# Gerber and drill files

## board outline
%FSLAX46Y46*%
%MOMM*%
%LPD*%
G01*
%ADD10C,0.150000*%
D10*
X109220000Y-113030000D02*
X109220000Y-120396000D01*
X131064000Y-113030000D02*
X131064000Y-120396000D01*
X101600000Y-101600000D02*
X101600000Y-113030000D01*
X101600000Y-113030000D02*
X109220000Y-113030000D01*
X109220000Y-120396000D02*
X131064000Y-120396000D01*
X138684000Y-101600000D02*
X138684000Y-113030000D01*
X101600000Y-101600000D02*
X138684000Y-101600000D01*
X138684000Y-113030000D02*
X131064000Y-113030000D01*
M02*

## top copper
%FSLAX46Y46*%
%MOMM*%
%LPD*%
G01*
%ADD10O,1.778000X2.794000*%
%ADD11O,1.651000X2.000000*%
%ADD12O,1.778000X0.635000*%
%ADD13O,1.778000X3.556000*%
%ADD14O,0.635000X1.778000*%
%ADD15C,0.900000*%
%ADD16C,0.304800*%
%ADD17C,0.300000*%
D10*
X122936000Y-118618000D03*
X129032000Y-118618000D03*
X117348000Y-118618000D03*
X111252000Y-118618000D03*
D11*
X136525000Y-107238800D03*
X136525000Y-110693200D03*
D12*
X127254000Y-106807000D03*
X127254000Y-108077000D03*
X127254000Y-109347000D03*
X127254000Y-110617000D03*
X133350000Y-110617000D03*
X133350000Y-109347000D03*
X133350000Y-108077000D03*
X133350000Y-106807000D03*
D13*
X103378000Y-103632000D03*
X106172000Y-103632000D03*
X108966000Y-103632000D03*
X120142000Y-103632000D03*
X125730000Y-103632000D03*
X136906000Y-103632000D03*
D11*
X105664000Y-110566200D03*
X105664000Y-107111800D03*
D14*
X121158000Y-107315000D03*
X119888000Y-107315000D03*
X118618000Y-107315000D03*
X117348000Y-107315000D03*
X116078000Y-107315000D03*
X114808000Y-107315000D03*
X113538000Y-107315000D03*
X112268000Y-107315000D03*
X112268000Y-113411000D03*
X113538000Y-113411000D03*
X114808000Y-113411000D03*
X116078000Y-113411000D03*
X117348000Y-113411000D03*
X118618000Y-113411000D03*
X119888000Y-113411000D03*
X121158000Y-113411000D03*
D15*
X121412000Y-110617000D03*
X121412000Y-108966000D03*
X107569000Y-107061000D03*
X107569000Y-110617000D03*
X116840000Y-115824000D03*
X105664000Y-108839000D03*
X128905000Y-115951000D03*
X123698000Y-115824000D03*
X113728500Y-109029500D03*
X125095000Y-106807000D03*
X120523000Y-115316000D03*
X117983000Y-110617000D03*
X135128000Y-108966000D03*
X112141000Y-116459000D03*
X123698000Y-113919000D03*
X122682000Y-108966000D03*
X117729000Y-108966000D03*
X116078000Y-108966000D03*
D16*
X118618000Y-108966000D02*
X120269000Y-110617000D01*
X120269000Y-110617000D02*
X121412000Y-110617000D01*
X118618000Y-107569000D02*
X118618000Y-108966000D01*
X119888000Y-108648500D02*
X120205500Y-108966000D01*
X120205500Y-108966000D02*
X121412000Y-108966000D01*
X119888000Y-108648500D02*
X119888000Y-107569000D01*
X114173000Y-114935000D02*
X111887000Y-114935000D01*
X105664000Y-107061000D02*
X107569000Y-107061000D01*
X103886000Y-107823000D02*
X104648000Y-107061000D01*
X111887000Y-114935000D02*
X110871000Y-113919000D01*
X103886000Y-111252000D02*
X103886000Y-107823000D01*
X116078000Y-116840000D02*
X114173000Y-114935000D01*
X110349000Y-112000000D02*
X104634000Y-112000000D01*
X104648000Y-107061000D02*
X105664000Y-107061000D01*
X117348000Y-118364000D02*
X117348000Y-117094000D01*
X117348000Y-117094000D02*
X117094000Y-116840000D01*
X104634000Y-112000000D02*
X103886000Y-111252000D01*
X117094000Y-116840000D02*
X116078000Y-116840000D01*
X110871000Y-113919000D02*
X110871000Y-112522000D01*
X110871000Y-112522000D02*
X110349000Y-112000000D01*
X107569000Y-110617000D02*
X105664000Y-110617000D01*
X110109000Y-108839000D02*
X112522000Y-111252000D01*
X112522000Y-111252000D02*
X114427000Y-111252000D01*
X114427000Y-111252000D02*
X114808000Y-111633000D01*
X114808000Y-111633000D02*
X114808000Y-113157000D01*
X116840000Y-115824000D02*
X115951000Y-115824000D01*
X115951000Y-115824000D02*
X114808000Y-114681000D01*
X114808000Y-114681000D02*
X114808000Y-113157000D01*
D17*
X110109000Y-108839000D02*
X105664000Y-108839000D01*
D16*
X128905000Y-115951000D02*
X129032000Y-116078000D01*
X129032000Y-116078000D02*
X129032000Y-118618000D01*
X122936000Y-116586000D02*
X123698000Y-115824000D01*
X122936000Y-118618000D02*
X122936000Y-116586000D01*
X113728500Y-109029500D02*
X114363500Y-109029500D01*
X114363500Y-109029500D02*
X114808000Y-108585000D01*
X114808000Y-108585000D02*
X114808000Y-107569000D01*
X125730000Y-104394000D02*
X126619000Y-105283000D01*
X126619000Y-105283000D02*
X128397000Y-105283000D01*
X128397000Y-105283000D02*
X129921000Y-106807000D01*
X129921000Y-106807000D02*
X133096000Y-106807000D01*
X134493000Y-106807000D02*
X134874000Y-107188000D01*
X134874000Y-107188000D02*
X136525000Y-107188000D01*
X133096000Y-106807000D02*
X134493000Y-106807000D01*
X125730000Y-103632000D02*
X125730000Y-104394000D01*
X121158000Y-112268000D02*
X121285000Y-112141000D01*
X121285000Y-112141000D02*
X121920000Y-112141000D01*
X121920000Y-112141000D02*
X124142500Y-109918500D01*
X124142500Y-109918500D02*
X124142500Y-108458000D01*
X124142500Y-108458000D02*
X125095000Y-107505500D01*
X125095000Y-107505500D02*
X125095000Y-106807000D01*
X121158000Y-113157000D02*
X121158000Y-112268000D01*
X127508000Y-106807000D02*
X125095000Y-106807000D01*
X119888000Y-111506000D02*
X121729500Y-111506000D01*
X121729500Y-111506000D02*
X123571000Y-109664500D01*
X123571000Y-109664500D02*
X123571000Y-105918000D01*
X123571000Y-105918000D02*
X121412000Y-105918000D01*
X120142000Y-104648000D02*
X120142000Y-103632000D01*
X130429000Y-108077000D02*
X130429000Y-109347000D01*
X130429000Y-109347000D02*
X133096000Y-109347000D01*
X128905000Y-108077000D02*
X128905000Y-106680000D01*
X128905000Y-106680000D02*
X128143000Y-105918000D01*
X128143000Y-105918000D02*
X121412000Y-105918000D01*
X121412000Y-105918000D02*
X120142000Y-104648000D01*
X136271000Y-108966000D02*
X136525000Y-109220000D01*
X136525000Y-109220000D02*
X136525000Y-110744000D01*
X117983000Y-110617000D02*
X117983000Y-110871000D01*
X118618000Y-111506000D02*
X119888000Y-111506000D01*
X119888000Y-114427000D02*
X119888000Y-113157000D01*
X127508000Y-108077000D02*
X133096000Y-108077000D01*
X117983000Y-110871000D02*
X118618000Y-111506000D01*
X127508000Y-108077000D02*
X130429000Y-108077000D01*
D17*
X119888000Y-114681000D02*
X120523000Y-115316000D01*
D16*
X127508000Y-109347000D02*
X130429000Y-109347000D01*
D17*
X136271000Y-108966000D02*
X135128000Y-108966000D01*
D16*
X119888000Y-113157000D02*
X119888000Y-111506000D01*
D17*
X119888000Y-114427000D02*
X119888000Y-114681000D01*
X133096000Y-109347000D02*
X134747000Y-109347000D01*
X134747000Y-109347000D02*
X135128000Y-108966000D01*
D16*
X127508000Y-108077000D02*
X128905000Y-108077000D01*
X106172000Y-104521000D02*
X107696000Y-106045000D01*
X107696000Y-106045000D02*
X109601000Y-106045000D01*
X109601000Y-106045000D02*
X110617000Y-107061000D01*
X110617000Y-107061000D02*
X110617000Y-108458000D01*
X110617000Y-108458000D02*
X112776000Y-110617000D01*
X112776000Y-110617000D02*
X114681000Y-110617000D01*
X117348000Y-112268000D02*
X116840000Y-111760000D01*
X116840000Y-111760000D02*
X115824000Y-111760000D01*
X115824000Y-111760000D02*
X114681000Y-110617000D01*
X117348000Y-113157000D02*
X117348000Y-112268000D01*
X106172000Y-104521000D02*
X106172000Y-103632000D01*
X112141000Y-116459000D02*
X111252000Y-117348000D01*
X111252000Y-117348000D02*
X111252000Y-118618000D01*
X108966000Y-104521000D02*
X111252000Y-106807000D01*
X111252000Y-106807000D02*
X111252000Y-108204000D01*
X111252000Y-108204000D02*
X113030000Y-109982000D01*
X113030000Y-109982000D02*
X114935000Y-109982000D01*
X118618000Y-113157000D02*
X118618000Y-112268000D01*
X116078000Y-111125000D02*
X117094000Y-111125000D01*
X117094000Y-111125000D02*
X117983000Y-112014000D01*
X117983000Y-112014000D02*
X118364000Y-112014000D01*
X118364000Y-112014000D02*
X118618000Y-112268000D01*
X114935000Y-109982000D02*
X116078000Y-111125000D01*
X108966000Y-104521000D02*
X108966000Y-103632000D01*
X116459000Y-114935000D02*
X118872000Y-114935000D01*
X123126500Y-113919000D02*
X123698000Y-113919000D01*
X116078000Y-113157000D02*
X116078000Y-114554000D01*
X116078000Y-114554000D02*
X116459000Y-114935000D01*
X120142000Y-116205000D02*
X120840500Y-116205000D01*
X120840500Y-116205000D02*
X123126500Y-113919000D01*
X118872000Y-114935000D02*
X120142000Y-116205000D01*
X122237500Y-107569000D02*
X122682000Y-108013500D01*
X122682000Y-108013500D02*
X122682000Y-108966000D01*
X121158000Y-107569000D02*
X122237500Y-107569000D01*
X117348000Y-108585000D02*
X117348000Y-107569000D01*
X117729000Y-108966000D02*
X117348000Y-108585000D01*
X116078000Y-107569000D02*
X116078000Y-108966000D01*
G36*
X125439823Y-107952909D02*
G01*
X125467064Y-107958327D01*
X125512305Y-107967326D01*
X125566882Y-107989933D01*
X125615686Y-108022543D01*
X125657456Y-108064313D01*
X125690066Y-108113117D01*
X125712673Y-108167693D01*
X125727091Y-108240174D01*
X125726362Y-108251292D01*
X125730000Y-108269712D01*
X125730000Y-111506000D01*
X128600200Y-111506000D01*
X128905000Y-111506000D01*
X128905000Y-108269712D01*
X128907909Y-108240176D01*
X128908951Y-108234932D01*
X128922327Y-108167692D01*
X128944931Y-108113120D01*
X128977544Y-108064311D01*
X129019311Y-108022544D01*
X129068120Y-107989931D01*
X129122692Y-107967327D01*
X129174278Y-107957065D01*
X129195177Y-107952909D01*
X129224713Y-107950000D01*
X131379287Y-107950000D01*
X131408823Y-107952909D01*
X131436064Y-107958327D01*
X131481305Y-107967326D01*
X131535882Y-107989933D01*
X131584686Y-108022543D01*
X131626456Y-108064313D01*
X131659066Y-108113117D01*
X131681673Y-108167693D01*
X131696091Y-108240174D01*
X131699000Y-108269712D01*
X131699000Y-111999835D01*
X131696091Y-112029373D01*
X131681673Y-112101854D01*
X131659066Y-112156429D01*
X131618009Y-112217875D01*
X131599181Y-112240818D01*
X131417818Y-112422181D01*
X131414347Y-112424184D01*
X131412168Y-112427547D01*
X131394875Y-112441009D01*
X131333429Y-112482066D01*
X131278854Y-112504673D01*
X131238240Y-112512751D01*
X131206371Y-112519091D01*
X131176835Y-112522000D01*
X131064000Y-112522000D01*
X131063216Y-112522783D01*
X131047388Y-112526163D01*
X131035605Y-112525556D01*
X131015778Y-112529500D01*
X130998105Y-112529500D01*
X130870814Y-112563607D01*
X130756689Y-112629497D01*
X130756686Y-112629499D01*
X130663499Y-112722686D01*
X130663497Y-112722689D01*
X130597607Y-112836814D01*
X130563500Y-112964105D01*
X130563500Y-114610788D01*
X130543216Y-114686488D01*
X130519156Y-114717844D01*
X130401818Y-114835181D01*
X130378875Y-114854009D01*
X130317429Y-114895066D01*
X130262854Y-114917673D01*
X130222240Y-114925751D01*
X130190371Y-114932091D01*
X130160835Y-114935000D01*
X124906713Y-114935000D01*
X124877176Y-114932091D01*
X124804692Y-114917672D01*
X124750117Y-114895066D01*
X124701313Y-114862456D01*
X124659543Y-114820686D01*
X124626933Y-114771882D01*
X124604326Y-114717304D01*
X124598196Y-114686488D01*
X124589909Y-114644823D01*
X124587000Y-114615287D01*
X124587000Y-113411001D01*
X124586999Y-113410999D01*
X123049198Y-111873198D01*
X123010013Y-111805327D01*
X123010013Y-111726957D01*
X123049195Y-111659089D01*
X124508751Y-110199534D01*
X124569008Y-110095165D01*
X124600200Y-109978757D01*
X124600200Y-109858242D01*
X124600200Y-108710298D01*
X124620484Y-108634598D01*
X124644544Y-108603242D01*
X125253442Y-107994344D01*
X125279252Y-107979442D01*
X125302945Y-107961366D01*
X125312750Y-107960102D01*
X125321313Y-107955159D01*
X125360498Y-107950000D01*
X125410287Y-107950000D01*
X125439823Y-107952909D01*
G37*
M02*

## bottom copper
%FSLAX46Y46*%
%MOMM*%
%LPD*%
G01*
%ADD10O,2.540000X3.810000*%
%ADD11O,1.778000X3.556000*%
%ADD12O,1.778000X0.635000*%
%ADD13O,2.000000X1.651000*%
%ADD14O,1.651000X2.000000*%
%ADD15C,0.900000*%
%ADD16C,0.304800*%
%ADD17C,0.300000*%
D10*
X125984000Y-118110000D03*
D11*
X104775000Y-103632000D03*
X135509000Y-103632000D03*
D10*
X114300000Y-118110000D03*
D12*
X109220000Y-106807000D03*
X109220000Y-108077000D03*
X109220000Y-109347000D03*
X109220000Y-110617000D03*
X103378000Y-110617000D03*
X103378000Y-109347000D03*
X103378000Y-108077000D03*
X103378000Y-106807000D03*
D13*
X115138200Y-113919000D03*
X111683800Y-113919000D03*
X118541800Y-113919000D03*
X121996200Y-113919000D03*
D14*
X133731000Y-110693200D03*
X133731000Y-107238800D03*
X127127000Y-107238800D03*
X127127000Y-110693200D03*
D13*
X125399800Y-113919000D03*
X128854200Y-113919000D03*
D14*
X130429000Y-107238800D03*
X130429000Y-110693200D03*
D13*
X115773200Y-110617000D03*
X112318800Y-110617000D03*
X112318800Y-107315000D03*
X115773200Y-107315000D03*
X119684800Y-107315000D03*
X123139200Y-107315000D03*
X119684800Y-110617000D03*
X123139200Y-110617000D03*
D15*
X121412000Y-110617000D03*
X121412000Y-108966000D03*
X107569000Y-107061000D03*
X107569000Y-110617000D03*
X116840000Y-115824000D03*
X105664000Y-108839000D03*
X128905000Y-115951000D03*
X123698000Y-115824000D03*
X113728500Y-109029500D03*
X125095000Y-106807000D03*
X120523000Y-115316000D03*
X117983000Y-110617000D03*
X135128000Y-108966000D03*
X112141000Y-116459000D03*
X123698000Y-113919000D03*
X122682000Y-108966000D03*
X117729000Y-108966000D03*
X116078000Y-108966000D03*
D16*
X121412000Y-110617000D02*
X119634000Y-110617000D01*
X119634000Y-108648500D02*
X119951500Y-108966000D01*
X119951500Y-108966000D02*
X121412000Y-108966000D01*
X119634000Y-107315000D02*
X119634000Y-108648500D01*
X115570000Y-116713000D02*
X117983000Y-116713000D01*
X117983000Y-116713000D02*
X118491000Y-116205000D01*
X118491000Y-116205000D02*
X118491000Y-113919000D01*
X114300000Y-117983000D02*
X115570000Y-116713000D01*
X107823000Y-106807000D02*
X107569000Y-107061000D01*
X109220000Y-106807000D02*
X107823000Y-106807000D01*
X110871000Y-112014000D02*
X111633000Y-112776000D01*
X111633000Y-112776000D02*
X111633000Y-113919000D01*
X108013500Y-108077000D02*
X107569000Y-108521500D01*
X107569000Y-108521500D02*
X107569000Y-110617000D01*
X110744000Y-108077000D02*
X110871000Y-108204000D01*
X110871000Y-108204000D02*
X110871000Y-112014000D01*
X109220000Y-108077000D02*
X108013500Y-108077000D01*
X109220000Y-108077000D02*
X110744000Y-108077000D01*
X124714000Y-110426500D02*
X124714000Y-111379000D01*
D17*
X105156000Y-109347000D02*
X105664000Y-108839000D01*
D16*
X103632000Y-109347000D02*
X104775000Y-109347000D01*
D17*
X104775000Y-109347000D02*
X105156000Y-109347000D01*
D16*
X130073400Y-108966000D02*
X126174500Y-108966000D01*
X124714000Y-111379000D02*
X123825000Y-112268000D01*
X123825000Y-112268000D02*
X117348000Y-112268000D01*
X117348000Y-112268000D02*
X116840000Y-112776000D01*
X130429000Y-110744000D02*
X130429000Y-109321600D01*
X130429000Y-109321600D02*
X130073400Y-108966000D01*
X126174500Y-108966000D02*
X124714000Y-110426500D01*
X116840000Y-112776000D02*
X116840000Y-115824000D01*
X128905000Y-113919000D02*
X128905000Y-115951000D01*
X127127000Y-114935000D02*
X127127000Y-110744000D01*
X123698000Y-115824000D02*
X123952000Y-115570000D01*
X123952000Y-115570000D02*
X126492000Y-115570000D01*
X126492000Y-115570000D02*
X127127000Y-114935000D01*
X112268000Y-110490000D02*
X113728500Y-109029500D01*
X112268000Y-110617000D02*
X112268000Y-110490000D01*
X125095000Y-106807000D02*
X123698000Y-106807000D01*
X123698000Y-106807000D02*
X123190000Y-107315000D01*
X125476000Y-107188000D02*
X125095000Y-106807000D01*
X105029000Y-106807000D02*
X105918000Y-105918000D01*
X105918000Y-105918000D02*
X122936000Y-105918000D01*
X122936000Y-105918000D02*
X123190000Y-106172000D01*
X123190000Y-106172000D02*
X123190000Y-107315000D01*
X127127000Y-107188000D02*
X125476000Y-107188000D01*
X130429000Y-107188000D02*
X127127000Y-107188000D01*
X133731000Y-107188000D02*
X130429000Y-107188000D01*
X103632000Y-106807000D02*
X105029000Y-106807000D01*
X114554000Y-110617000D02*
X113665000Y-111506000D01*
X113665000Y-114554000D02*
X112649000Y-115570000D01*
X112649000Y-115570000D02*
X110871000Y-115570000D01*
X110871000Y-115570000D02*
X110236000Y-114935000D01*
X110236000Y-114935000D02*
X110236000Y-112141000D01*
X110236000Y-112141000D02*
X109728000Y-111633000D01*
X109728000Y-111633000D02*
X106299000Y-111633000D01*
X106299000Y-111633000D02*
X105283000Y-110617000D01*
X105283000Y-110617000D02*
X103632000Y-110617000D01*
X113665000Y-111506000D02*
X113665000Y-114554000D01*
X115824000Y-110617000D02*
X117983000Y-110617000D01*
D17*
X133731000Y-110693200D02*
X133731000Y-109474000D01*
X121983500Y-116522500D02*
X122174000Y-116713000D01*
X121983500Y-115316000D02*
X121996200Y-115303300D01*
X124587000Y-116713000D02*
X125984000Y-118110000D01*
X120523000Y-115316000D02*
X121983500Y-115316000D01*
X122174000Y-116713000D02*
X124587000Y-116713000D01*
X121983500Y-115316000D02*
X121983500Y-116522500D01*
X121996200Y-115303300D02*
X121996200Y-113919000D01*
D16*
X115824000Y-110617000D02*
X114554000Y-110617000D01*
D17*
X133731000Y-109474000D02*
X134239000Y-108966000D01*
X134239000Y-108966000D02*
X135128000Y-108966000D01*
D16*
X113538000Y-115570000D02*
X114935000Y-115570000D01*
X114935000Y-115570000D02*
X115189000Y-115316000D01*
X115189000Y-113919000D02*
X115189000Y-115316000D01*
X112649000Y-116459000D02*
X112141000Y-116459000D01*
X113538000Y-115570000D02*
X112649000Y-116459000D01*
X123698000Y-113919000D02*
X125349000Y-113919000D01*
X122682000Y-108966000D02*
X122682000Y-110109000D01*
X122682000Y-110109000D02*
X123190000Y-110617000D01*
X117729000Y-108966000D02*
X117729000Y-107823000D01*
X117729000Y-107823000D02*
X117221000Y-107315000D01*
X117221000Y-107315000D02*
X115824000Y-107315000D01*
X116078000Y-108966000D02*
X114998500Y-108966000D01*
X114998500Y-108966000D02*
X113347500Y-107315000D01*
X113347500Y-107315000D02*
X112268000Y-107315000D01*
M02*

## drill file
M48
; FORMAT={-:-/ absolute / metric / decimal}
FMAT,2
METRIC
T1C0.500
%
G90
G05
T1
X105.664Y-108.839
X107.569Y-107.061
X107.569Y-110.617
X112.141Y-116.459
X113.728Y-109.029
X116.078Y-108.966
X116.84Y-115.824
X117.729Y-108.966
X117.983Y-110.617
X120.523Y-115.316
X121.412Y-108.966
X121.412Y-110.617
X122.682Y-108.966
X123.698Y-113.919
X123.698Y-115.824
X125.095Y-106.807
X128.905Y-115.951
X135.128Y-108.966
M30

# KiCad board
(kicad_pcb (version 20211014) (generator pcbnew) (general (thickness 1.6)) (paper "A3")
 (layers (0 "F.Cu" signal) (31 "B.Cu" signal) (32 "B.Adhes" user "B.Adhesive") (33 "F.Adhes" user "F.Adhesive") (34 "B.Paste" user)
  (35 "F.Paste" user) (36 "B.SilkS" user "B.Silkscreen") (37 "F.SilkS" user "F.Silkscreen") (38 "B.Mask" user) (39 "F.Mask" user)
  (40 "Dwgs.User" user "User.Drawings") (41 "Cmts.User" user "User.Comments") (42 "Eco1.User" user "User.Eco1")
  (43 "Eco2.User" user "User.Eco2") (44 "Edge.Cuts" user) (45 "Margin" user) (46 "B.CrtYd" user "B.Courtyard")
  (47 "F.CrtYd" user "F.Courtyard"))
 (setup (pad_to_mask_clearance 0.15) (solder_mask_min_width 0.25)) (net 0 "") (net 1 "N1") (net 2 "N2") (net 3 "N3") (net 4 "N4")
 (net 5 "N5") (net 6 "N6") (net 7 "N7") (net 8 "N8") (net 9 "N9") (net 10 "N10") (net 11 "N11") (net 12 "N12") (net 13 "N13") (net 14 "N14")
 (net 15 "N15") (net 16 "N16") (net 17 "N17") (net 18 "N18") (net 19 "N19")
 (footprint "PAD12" (layer "F.Cu") (at 125.984 118.11)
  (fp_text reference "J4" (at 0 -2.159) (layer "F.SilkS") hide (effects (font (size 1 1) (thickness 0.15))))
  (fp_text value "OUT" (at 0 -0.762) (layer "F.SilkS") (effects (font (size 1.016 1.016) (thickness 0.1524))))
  (pad "1" smd oval locked (at 0 0) (size 2.54 3.81) (layers "B.Cu" "B.Mask") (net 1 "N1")))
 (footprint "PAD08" (layer "F.Cu") (at 122.936 118.618)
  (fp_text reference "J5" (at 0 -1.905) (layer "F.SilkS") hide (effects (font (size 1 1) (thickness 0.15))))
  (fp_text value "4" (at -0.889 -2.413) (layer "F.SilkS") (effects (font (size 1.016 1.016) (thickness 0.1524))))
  (pad "1" smd oval locked (at 0 0) (size 1.778 2.794) (layers "F.Cu" "F.Paste" "F.Mask") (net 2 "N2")))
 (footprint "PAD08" (layer "F.Cu") (at 129.032 118.618)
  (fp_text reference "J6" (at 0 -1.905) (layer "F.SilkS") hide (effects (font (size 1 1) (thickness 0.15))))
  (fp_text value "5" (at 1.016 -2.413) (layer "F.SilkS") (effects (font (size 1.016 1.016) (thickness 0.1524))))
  (pad "1" smd oval locked (at 0 0) (size 1.778 2.794) (layers "F.Cu" "F.Paste" "F.Mask") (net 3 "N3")))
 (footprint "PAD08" (layer "F.Cu") (at 117.348 118.618)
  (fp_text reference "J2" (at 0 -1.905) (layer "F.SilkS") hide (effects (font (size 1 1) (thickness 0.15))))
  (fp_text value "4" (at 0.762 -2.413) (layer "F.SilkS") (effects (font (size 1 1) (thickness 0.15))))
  (pad "1" smd oval locked (at 0 0) (size 1.778 2.794) (layers "F.Cu" "F.Paste" "F.Mask") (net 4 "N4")))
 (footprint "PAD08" (layer "F.Cu") (at 111.252 118.618)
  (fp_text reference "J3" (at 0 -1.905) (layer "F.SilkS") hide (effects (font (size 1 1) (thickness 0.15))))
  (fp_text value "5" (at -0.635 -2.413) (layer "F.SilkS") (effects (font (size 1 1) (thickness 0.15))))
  (pad "1" smd oval locked (at 0 0) (size 1.778 2.794) (layers "F.Cu" "F.Paste" "F.Mask") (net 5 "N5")))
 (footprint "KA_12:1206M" (layer "F.Cu") (at 136.525 108.966 -90)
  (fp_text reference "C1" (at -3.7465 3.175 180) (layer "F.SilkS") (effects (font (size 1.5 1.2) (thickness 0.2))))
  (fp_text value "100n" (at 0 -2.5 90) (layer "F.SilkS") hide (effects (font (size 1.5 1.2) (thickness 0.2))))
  (pad "1" smd oval locked (at -1.7272 0 270) (size 2 1.651) (layers "F.Cu" "F.Paste" "F.Mask") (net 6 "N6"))
  (pad "2" smd oval locked (at 1.7272 0 270) (size 2 1.651) (layers "F.Cu" "F.Paste" "F.Mask") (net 1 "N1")))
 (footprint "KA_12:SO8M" (layer "F.Cu") (at 130.302 108.712 -90)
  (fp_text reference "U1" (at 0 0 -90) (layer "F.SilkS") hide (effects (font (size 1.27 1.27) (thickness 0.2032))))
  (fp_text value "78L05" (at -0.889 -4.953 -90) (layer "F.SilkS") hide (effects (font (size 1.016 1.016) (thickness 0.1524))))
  (pad "1" smd oval (at -1.905 2.794 270) (size 0.635 1.778) (drill (offset 0 0.254)) (layers "F.Cu" "F.Paste" "F.Mask") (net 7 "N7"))
  (pad "2" smd oval (at -0.635 2.794 270) (size 0.635 1.778) (drill (offset 0 0.254)) (layers "F.Cu" "F.Paste" "F.Mask") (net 1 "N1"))
  (pad "3" smd oval (at 0.635 2.794 270) (size 0.635 1.778) (drill (offset 0 0.254)) (layers "F.Cu" "F.Paste" "F.Mask") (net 1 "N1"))
  (pad "4" smd oval (at 1.905 2.794 270) (size 0.635 1.778) (drill (offset 0 0.254)) (layers "F.Cu" "F.Paste" "F.Mask"))
  (pad "5" smd oval (at 1.905 -2.794 270) (size 0.635 1.778) (drill (offset 0 -0.254)) (layers "F.Cu" "F.Paste" "F.Mask"))
  (pad "6" smd oval (at 0.635 -2.794 270) (size 0.635 1.778) (drill (offset 0 -0.254)) (layers "F.Cu" "F.Paste" "F.Mask") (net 1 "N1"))
  (pad "7" smd oval (at -0.635 -2.794 270) (size 0.635 1.778) (drill (offset 0 -0.254)) (layers "F.Cu" "F.Paste" "F.Mask") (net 1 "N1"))
  (pad "8" smd oval (at -1.905 -2.794 270) (size 0.635 1.778) (drill (offset 0 -0.254)) (layers "F.Cu" "F.Paste" "F.Mask") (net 6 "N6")))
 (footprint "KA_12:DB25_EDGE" (layer "F.Cu") (at 120.142 103.632)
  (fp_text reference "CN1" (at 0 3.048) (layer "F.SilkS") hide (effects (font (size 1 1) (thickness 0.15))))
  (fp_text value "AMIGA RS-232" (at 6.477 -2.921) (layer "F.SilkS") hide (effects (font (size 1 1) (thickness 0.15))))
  (pad "1" smd oval locked (at -16.764 0) (size 1.778 3.556) (layers "F.Cu" "F.Paste" "F.Mask"))
  (pad "2" smd oval locked (at -13.97 0) (size 1.778 3.556) (layers "F.Cu" "F.Paste" "F.Mask") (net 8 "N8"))
  (pad "3" smd oval locked (at -11.176 0) (size 1.778 3.556) (layers "F.Cu" "F.Paste" "F.Mask") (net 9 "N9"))
  (pad "7" smd oval locked (at 0 0) (size 1.778 3.556) (layers "F.Cu" "F.Paste" "F.Mask") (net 1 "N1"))
  (pad "9" smd oval locked (at 5.588 0) (size 1.778 3.556) (layers "F.Cu" "F.Paste" "F.Mask") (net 6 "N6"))
  (pad "13" smd oval locked (at 16.764 0) (size 1.778 3.556) (layers "F.Cu" "F.Paste" "F.Mask"))
  (pad "14" smd oval locked (at -15.367 0) (size 1.778 3.556) (layers "B.Cu" "B.Paste" "B.Mask"))
  (pad "25" smd oval locked (at 15.367 0) (size 1.778 3.556) (layers "B.Cu" "B.Paste" "B.Mask")))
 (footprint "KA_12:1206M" (layer "F.Cu") (at 105.664 108.839 90)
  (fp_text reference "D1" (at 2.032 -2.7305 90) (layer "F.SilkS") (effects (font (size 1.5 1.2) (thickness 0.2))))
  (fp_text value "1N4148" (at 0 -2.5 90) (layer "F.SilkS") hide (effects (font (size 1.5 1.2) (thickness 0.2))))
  (pad "1" smd oval locked (at -1.7272 0 90) (size 2 1.651) (layers "F.Cu" "F.Paste" "F.Mask") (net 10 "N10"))
  (pad "2" smd oval locked (at 1.7272 0 90) (size 2 1.651) (layers "F.Cu" "F.Paste" "F.Mask") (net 4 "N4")))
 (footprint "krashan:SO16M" (layer "F.Cu") (at 116.713 110.363 180)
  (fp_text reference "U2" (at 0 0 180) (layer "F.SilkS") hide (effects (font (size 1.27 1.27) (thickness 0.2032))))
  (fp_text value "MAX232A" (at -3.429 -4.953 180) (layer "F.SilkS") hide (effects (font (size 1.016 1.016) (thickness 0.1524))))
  (pad "1" smd oval (at -4.445 2.794 180) (size 0.635 1.778) (drill (offset 0 0.254)) (layers "F.Cu" "F.Paste" "F.Mask") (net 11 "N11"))
  (pad "2" smd oval (at -3.175 2.794 180) (size 0.635 1.778) (drill (offset 0 0.254)) (layers "F.Cu" "F.Paste" "F.Mask") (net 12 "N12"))
  (pad "3" smd oval (at -1.905 2.794 180) (size 0.635 1.778) (drill (offset 0 0.254)) (layers "F.Cu" "F.Paste" "F.Mask") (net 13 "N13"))
  (pad "4" smd oval (at -0.635 2.794 180) (size 0.635 1.778) (drill (offset 0 0.254)) (layers "F.Cu" "F.Paste" "F.Mask") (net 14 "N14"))
  (pad "5" smd oval (at 0.635 2.794 180) (size 0.635 1.778) (drill (offset 0 0.254)) (layers "F.Cu" "F.Paste" "F.Mask") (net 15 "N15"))
  (pad "6" smd oval (at 1.905 2.794 180) (size 0.635 1.778) (drill (offset 0 0.254)) (layers "F.Cu" "F.Paste" "F.Mask") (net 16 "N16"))
  (pad "7" smd oval (at 3.175 2.794 180) (size 0.635 1.778) (drill (offset 0 0.254)) (layers "F.Cu" "F.Paste" "F.Mask"))
  (pad "8" smd oval (at 4.445 2.794 180) (size 0.635 1.778) (drill (offset 0 0.254)) (layers "F.Cu" "F.Paste" "F.Mask"))
  (pad "9" smd oval (at 4.445 -2.794 180) (size 0.635 1.778) (drill (offset 0 -0.254)) (layers "F.Cu" "F.Paste" "F.Mask"))
  (pad "10" smd oval (at 3.175 -2.794 180) (size 0.635 1.778) (drill (offset 0 -0.254)) (layers "F.Cu" "F.Paste" "F.Mask"))
  (pad "11" smd oval (at 1.905 -2.794 180) (size 0.635 1.778) (drill (offset 0 -0.254)) (layers "F.Cu" "F.Paste" "F.Mask") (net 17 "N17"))
  (pad "12" smd oval (at 0.635 -2.794 180) (size 0.635 1.778) (drill (offset 0 -0.254)) (layers "F.Cu" "F.Paste" "F.Mask") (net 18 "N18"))
  (pad "13" smd oval (at -0.635 -2.794 180) (size 0.635 1.778) (drill (offset 0 -0.254)) (layers "F.Cu" "F.Paste" "F.Mask") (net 8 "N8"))
  (pad "14" smd oval (at -1.905 -2.794 180) (size 0.635 1.778) (drill (offset 0 -0.254)) (layers "F.Cu" "F.Paste" "F.Mask") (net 9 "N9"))
  (pad "15" smd oval (at -3.175 -2.794 180) (size 0.635 1.778) (drill (offset 0 -0.254)) (layers "F.Cu" "F.Paste" "F.Mask") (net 1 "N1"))
  (pad "16" smd oval (at -4.445 -2.794 180) (size 0.635 1.778) (drill (offset 0 -0.254)) (layers "F.Cu" "F.Paste" "F.Mask") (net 7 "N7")))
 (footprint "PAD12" (layer "F.Cu") (at 114.3 118.11)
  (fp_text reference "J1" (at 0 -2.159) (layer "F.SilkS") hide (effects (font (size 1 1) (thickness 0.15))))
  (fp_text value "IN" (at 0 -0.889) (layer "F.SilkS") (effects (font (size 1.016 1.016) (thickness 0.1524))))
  (pad "1" smd oval locked (at 0 0) (size 2.54 3.81) (layers "B.Cu" "B.Mask") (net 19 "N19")))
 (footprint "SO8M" (layer "B.Cu") (at 106.426 108.712 -90)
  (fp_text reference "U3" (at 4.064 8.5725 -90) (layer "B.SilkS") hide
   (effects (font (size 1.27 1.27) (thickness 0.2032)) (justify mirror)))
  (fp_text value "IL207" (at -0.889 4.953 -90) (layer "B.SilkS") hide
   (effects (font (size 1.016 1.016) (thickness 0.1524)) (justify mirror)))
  (pad "1" smd oval locked (at -1.905 -2.794 270) (size 0.635 1.778) (layers "B.Cu" "B.Paste" "B.Mask") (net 4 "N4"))
  (pad "2" smd oval locked (at -0.635 -2.794 270) (size 0.635 1.778) (layers "B.Cu" "B.Paste" "B.Mask") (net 10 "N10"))
  (pad "3" smd oval locked (at 0.635 -2.794 270) (size 0.635 1.778) (layers "B.Cu" "B.Paste" "B.Mask"))
  (pad "4" smd oval locked (at 1.905 -2.794 270) (size 0.635 1.778) (layers "B.Cu" "B.Paste" "B.Mask"))
  (pad "5" smd oval locked (at 1.905 2.794 270) (size 0.635 1.778) (drill (offset 0 0.254)) (layers "B.Cu" "B.Paste" "B.Mask") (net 1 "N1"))
  (pad "6" smd oval locked (at 0.635 2.794 270) (size 0.635 1.778) (drill (offset 0 0.254)) (layers "B.Cu" "B.Paste" "B.Mask")
   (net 17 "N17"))
  (pad "7" smd oval locked (at -0.635 2.794 270) (size 0.635 1.778) (drill (offset 0 0.254)) (layers "B.Cu" "B.Paste" "B.Mask"))
  (pad "8" smd oval locked (at -1.905 2.794 270) (size 0.635 1.778) (drill (offset 0 0.254)) (layers "B.Cu" "B.Paste" "B.Mask") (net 7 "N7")))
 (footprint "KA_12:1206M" (layer "B.Cu") (at 113.411 113.919 180)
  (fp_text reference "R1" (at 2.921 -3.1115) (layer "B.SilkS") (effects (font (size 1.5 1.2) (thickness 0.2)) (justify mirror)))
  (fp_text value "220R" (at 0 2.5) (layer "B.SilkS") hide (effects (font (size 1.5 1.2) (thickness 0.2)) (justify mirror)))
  (pad "1" smd oval locked (at -1.7272 0 180) (size 2 1.651) (layers "B.Cu" "B.Paste" "B.Mask") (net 5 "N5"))
  (pad "2" smd oval locked (at 1.7272 0 180) (size 2 1.651) (layers "B.Cu" "B.Paste" "B.Mask") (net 10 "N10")))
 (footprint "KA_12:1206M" (layer "B.Cu") (at 120.269 113.919)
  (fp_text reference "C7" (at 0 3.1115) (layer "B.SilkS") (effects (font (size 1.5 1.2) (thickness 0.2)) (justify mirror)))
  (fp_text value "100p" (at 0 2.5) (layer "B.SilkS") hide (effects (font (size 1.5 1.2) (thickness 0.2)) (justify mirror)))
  (pad "1" smd oval locked (at -1.7272 0) (size 2 1.651) (layers "B.Cu" "B.Paste" "B.Mask") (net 19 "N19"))
  (pad "2" smd oval locked (at 1.7272 0) (size 2 1.651) (layers "B.Cu" "B.Paste" "B.Mask") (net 1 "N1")))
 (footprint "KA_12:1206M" (layer "B.Cu") (at 133.731 108.966 90)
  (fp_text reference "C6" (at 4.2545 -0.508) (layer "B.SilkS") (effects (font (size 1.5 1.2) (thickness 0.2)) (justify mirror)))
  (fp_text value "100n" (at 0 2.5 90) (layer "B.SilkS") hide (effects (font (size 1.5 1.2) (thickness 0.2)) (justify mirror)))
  (pad "1" smd oval locked (at -1.7272 0 90) (size 2 1.651) (layers "B.Cu" "B.Paste" "B.Mask") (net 1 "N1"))
  (pad "2" smd oval locked (at 1.7272 0 90) (size 2 1.651) (layers "B.Cu" "B.Paste" "B.Mask") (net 7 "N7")))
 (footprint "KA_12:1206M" (layer "B.Cu") (at 127.127 108.966 -90)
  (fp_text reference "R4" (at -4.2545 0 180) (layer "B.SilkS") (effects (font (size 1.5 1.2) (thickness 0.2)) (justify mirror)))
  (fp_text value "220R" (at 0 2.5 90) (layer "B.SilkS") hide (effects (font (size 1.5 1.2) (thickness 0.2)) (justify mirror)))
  (pad "1" smd oval locked (at -1.7272 0 270) (size 2 1.651) (layers "B.Cu" "B.Paste" "B.Mask") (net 7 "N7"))
  (pad "2" smd oval locked (at 1.7272 0 270) (size 2 1.651) (layers "B.Cu" "B.Paste" "B.Mask") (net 2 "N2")))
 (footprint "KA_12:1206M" (layer "B.Cu") (at 127.127 113.919)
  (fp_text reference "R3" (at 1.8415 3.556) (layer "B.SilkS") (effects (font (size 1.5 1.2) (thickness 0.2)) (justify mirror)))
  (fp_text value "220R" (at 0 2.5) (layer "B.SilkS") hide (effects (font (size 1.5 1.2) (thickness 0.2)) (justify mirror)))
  (pad "1" smd oval locked (at -1.7272 0) (size 2 1.651) (layers "B.Cu" "B.Paste" "B.Mask") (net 18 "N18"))
  (pad "2" smd oval locked (at 1.7272 0) (size 2 1.651) (layers "B.Cu" "B.Paste" "B.Mask") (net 3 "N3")))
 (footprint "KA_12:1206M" (layer "B.Cu") (at 130.429 108.966 -90)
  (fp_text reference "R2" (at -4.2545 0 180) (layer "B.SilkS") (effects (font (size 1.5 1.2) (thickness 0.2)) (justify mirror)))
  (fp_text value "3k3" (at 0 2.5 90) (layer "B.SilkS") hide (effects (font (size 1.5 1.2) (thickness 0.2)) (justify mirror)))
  (pad "1" smd oval locked (at -1.7272 0 270) (size 2 1.651) (layers "B.Cu" "B.Paste" "B.Mask") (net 7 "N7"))
  (pad "2" smd oval locked (at 1.7272 0 270) (size 2 1.651) (layers "B.Cu" "B.Paste" "B.Mask") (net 17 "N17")))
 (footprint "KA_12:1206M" (layer "B.Cu") (at 114.046 110.617 180)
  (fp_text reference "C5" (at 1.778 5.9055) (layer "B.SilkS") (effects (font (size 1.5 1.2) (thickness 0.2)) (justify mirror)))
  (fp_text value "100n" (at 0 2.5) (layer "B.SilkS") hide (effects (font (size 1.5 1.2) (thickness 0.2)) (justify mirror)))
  (pad "1" smd oval locked (at -1.7272 0 180) (size 2 1.651) (layers "B.Cu" "B.Paste" "B.Mask") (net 1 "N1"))
  (pad "2" smd oval locked (at 1.7272 0 180) (size 2 1.651) (layers "B.Cu" "B.Paste" "B.Mask") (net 16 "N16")))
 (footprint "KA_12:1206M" (layer "B.Cu") (at 114.046 107.315)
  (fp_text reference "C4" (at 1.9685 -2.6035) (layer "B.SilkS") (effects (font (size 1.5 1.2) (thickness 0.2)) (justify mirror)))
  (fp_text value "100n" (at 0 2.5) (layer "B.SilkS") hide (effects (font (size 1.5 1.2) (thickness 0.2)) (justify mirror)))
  (pad "1" smd oval locked (at -1.7272 0) (size 2 1.651) (layers "B.Cu" "B.Paste" "B.Mask") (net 15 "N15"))
  (pad "2" smd oval locked (at 1.7272 0) (size 2 1.651) (layers "B.Cu" "B.Paste" "B.Mask") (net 14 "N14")))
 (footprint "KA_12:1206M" (layer "B.Cu") (at 121.412 107.315)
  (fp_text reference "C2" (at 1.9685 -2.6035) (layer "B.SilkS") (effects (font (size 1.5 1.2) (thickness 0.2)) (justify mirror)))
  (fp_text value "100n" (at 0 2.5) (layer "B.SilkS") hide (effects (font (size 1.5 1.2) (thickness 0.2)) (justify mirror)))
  (pad "1" smd oval locked (at -1.7272 0) (size 2 1.651) (layers "B.Cu" "B.Paste" "B.Mask") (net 12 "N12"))
  (pad "2" smd oval locked (at 1.7272 0) (size 2 1.651) (layers "B.Cu" "B.Paste" "B.Mask") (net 7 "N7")))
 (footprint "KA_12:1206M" (layer "B.Cu") (at 121.412 110.617)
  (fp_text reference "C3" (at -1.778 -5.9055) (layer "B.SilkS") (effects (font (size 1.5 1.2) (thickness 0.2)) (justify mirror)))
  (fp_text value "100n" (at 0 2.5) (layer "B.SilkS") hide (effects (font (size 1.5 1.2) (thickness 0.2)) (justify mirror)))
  (pad "1" smd oval locked (at -1.7272 0) (size 2 1.651) (layers "B.Cu" "B.Paste" "B.Mask") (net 13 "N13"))
  (pad "2" smd oval locked (at 1.7272 0) (size 2 1.651) (layers "B.Cu" "B.Paste" "B.Mask") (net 11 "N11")))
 (gr_line (start 109.22 113.03) (end 109.22 120.396) (layer "Edge.Cuts") (width 0.15))
 (gr_line (start 131.064 113.03) (end 131.064 120.396) (layer "Edge.Cuts") (width 0.15))
 (gr_line (start 101.6 101.6) (end 101.6 113.03) (layer "Edge.Cuts") (width 0.15))
 (gr_line (start 101.6 113.03) (end 109.22 113.03) (layer "Edge.Cuts") (width 0.15))
 (gr_line (start 109.22 120.396) (end 131.064 120.396) (layer "Edge.Cuts") (width 0.15))
 (gr_line (start 138.684 101.6) (end 138.684 113.03) (layer "Edge.Cuts") (width 0.15))
 (gr_line (start 101.6 101.6) (end 138.684 101.6) (layer "Edge.Cuts") (width 0.15))
 (gr_line (start 138.684 113.03) (end 131.064 113.03) (layer "Edge.Cuts") (width 0.15))
 (segment (start 118.618 108.966) (end 120.269 110.617) (width 0.3048) (layer "F.Cu") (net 13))
 (segment (start 120.269 110.617) (end 121.412 110.617) (width 0.3048) (layer "F.Cu") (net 13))
 (segment (start 118.618 107.569) (end 118.618 108.966) (width 0.3048) (layer "F.Cu") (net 13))
 (via (at 121.412 110.617) (size 0.9) (drill 0.5) (layers "F.Cu" "B.Cu") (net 13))
 (segment (start 121.412 110.617) (end 119.634 110.617) (width 0.3048) (layer "B.Cu") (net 13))
 (segment (start 119.888 108.6485) (end 120.2055 108.966) (width 0.3048) (layer "F.Cu") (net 12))
 (segment (start 120.2055 108.966) (end 121.412 108.966) (width 0.3048) (layer "F.Cu") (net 12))
 (segment (start 119.888 108.6485) (end 119.888 107.569) (width 0.3048) (layer "F.Cu") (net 12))
 (via (at 121.412 108.966) (size 0.9) (drill 0.5) (layers "F.Cu" "B.Cu") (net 12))
 (segment (start 119.634 108.6485) (end 119.9515 108.966) (width 0.3048) (layer "B.Cu") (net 12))
 (segment (start 119.9515 108.966) (end 121.412 108.966) (width 0.3048) (layer "B.Cu") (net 12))
 (segment (start 119.634 107.315) (end 119.634 108.6485) (width 0.3048) (layer "B.Cu") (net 12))
 (segment (start 115.57 116.713) (end 117.983 116.713) (width 0.3048) (layer "B.Cu") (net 19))
 (segment (start 117.983 116.713) (end 118.491 116.205) (width 0.3048) (layer "B.Cu") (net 19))
 (segment (start 118.491 116.205) (end 118.491 113.919) (width 0.3048) (layer "B.Cu") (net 19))
 (segment (start 114.3 117.983) (end 115.57 116.713) (width 0.3048) (layer "B.Cu") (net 19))
 (segment (start 114.173 114.935) (end 111.887 114.935) (width 0.3048) (layer "F.Cu") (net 4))
 (segment (start 105.664 107.061) (end 107.569 107.061) (width 0.3048) (layer "F.Cu") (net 4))
 (segment (start 103.886 107.823) (end 104.648 107.061) (width 0.3048) (layer "F.Cu") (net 4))
 (segment (start 111.887 114.935) (end 110.871 113.919) (width 0.3048) (layer "F.Cu") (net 4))
 (segment (start 103.886 111.252) (end 103.886 107.823) (width 0.3048) (layer "F.Cu") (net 4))
 (segment (start 116.078 116.84) (end 114.173 114.935) (width 0.3048) (layer "F.Cu") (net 4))
 (segment (start 110.349 112) (end 104.634 112) (width 0.3048) (layer "F.Cu") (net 4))
 (segment (start 104.648 107.061) (end 105.664 107.061) (width 0.3048) (layer "F.Cu") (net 4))
 (segment (start 117.348 118.364) (end 117.348 117.094) (width 0.3048) (layer "F.Cu") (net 4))
 (segment (start 117.348 117.094) (end 117.094 116.84) (width 0.3048) (layer "F.Cu") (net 4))
 (segment (start 104.634 112) (end 103.886 111.252) (width 0.3048) (layer "F.Cu") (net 4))
 (segment (start 117.094 116.84) (end 116.078 116.84) (width 0.3048) (layer "F.Cu") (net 4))
 (segment (start 110.871 113.919) (end 110.871 112.522) (width 0.3048) (layer "F.Cu") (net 4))
 (segment (start 110.871 112.522) (end 110.349 112) (width 0.3048) (layer "F.Cu") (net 4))
 (via (at 107.569 107.061) (size 0.9) (drill 0.5) (layers "F.Cu" "B.Cu") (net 4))
 (segment (start 107.823 106.807) (end 107.569 107.061) (width 0.3048) (layer "B.Cu") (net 4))
 (segment (start 109.22 106.807) (end 107.823 106.807) (width 0.3048) (layer "B.Cu") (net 4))
 (segment (start 107.569 110.617) (end 105.664 110.617) (width 0.3048) (layer "F.Cu") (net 10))
 (via (at 107.569 110.617) (size 0.9) (drill 0.5) (layers "F.Cu" "B.Cu") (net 10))
 (segment (start 110.871 112.014) (end 111.633 112.776) (width 0.3048) (layer "B.Cu") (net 10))
 (segment (start 111.633 112.776) (end 111.633 113.919) (width 0.3048) (layer "B.Cu") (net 10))
 (segment (start 108.0135 108.077) (end 107.569 108.5215) (width 0.3048) (layer "B.Cu") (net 10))
 (segment (start 107.569 108.5215) (end 107.569 110.617) (width 0.3048) (layer "B.Cu") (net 10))
 (segment (start 110.744 108.077) (end 110.871 108.204) (width 0.3048) (layer "B.Cu") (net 10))
 (segment (start 110.871 108.204) (end 110.871 112.014) (width 0.3048) (layer "B.Cu") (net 10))
 (segment (start 109.22 108.077) (end 108.0135 108.077) (width 0.3048) (layer "B.Cu") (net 10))
 (segment (start 109.22 108.077) (end 110.744 108.077) (width 0.3048) (layer "B.Cu") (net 10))
 (segment (start 110.109 108.839) (end 112.522 111.252) (width 0.3048) (layer "F.Cu") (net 17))
 (segment (start 112.522 111.252) (end 114.427 111.252) (width 0.3048) (layer "F.Cu") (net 17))
 (segment (start 114.427 111.252) (end 114.808 111.633) (width 0.3048) (layer "F.Cu") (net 17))
 (segment (start 114.808 111.633) (end 114.808 113.157) (width 0.3048) (layer "F.Cu") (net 17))
 (segment (start 116.84 115.824) (end 115.951 115.824) (width 0.3048) (layer "F.Cu") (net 17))
 (segment (start 115.951 115.824) (end 114.808 114.681) (width 0.3048) (layer "F.Cu") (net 17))
 (segment (start 114.808 114.681) (end 114.808 113.157) (width 0.3048) (layer "F.Cu") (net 17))
 (segment (start 110.109 108.839) (end 105.664 108.839) (width 0.3) (layer "F.Cu") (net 17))
 (via (at 116.84 115.824) (size 0.9) (drill 0.5) (layers "F.Cu" "B.Cu") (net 17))
 (via (at 105.664 108.839) (size 0.9) (drill 0.5) (layers "F.Cu" "B.Cu") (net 17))
 (segment (start 124.714 110.4265) (end 124.714 111.379) (width 0.3048) (layer "B.Cu") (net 17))
 (segment (start 105.156 109.347) (end 105.664 108.839) (width 0.3) (layer "B.Cu") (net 17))
 (segment (start 103.632 109.347) (end 104.775 109.347) (width 0.3048) (layer "B.Cu") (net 17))
 (segment (start 104.775 109.347) (end 105.156 109.347) (width 0.3) (layer "B.Cu") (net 17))
 (segment (start 130.0734 108.966) (end 126.1745 108.966) (width 0.3048) (layer "B.Cu") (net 17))
 (segment (start 124.714 111.379) (end 123.825 112.268) (width 0.3048) (layer "B.Cu") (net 17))
 (segment (start 123.825 112.268) (end 117.348 112.268) (width 0.3048) (layer "B.Cu") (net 17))
 (segment (start 117.348 112.268) (end 116.84 112.776) (width 0.3048) (layer "B.Cu") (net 17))
 (segment (start 130.429 110.744) (end 130.429 109.3216) (width 0.3048) (layer "B.Cu") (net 17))
 (segment (start 130.429 109.3216) (end 130.0734 108.966) (width 0.3048) (layer "B.Cu") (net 17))
 (segment (start 126.1745 108.966) (end 124.714 110.4265) (width 0.3048) (layer "B.Cu") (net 17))
 (segment (start 116.84 112.776) (end 116.84 115.824) (width 0.3048) (layer "B.Cu") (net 17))
 (segment (start 128.905 115.951) (end 129.032 116.078) (width 0.3048) (layer "F.Cu") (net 3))
 (segment (start 129.032 116.078) (end 129.032 118.618) (width 0.3048) (layer "F.Cu") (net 3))
 (via (at 128.905 115.951) (size 0.9) (drill 0.5) (layers "F.Cu" "B.Cu") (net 3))
 (segment (start 128.905 113.919) (end 128.905 115.951) (width 0.3048) (layer "B.Cu") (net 3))
 (segment (start 122.936 116.586) (end 123.698 115.824) (width 0.3048) (layer "F.Cu") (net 2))
 (segment (start 122.936 118.618) (end 122.936 116.586) (width 0.3048) (layer "F.Cu") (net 2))
 (via (at 123.698 115.824) (size 0.9) (drill 0.5) (layers "F.Cu" "B.Cu") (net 2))
 (segment (start 127.127 114.935) (end 127.127 110.744) (width 0.3048) (layer "B.Cu") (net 2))
 (segment (start 123.698 115.824) (end 123.952 115.57) (width 0.3048) (layer "B.Cu") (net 2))
 (segment (start 123.952 115.57) (end 126.492 115.57) (width 0.3048) (layer "B.Cu") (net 2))
 (segment (start 126.492 115.57) (end 127.127 114.935) (width 0.3048) (layer "B.Cu") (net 2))
 (segment (start 113.7285 109.0295) (end 114.3635 109.0295) (width 0.3048) (layer "F.Cu") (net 16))
 (segment (start 114.3635 109.0295) (end 114.808 108.585) (width 0.3048) (layer "F.Cu") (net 16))
 (segment (start 114.808 108.585) (end 114.808 107.569) (width 0.3048) (layer "F.Cu") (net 16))
 (via (at 113.7285 109.0295) (size 0.9) (drill 0.5) (layers "F.Cu" "B.Cu") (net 16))
 (segment (start 112.268 110.49) (end 113.7285 109.0295) (width 0.3048) (layer "B.Cu") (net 16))
 (segment (start 112.268 110.617) (end 112.268 110.49) (width 0.3048) (layer "B.Cu") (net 16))
 (segment (start 125.73 104.394) (end 126.619 105.283) (width 0.3048) (layer "F.Cu") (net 6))
 (segment (start 126.619 105.283) (end 128.397 105.283) (width 0.3048) (layer "F.Cu") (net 6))
 (segment (start 128.397 105.283) (end 129.921 106.807) (width 0.3048) (layer "F.Cu") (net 6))
 (segment (start 129.921 106.807) (end 133.096 106.807) (width 0.3048) (layer "F.Cu") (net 6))
 (segment (start 134.493 106.807) (end 134.874 107.188) (width 0.3048) (layer "F.Cu") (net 6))
 (segment (start 134.874 107.188) (end 136.525 107.188) (width 0.3048) (layer "F.Cu") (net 6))
 (segment (start 133.096 106.807) (end 134.493 106.807) (width 0.3048) (layer "F.Cu") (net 6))
 (segment (start 125.73 103.632) (end 125.73 104.394) (width 0.3048) (layer "F.Cu") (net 6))
 (segment (start 121.158 112.268) (end 121.285 112.141) (width 0.3048) (layer "F.Cu") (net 7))
 (segment (start 121.285 112.141) (end 121.92 112.141) (width 0.3048) (layer "F.Cu") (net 7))
 (segment (start 121.92 112.141) (end 124.1425 109.9185) (width 0.3048) (layer "F.Cu") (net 7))
 (segment (start 124.1425 109.9185) (end 124.1425 108.458) (width 0.3048) (layer "F.Cu") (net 7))
 (segment (start 124.1425 108.458) (end 125.095 107.5055) (width 0.3048) (layer "F.Cu") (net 7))
 (segment (start 125.095 107.5055) (end 125.095 106.807) (width 0.3048) (layer "F.Cu") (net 7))
 (segment (start 121.158 113.157) (end 121.158 112.268) (width 0.3048) (layer "F.Cu") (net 7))
 (segment (start 127.508 106.807) (end 125.095 106.807) (width 0.3048) (layer "F.Cu") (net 7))
 (via (at 125.095 106.807) (size 0.9) (drill 0.5) (layers "F.Cu" "B.Cu") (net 7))
 (segment (start 125.095 106.807) (end 123.698 106.807) (width 0.3048) (layer "B.Cu") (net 7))
 (segment (start 123.698 106.807) (end 123.19 107.315) (width 0.3048) (layer "B.Cu") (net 7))
 (segment (start 125.476 107.188) (end 125.095 106.807) (width 0.3048) (layer "B.Cu") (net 7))
 (segment (start 105.029 106.807) (end 105.918 105.918) (width 0.3048) (layer "B.Cu") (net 7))
 (segment (start 105.918 105.918) (end 122.936 105.918) (width 0.3048) (layer "B.Cu") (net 7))
 (segment (start 122.936 105.918) (end 123.19 106.172) (width 0.3048) (layer "B.Cu") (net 7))
 (segment (start 123.19 106.172) (end 123.19 107.315) (width 0.3048) (layer "B.Cu") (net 7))
 (segment (start 127.127 107.188) (end 125.476 107.188) (width 0.3048) (layer "B.Cu") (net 7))
 (segment (start 130.429 107.188) (end 127.127 107.188) (width 0.3048) (layer "B.Cu") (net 7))
 (segment (start 133.731 107.188) (end 130.429 107.188) (width 0.3048) (layer "B.Cu") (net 7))
 (segment (start 103.632 106.807) (end 105.029 106.807) (width 0.3048) (layer "B.Cu") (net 7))
 (segment (start 119.888 111.506) (end 121.7295 111.506) (width 0.3048) (layer "F.Cu") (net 1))
 (segment (start 121.7295 111.506) (end 123.571 109.6645) (width 0.3048) (layer "F.Cu") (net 1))
 (segment (start 123.571 109.6645) (end 123.571 105.918) (width 0.3048) (layer "F.Cu") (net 1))
 (segment (start 123.571 105.918) (end 121.412 105.918) (width 0.3048) (layer "F.Cu") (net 1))
 (segment (start 120.142 104.648) (end 120.142 103.632) (width 0.3048) (layer "F.Cu") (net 1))
 (segment (start 130.429 108.077) (end 130.429 109.347) (width 0.3048) (layer "F.Cu") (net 1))
 (segment (start 130.429 109.347) (end 133.096 109.347) (width 0.3048) (layer "F.Cu") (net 1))
 (segment (start 128.905 108.077) (end 128.905 106.68) (width 0.3048) (layer "F.Cu") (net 1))
 (segment (start 128.905 106.68) (end 128.143 105.918) (width 0.3048) (layer "F.Cu") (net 1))
 (segment (start 128.143 105.918) (end 121.412 105.918) (width 0.3048) (layer "F.Cu") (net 1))
 (segment (start 121.412 105.918) (end 120.142 104.648) (width 0.3048) (layer "F.Cu") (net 1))
 (segment (start 136.271 108.966) (end 136.525 109.22) (width 0.3048) (layer "F.Cu") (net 1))
 (segment (start 136.525 109.22) (end 136.525 110.744) (width 0.3048) (layer "F.Cu") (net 1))
 (segment (start 117.983 110.617) (end 117.983 110.871) (width 0.3048) (layer "F.Cu") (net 1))
 (segment (start 118.618 111.506) (end 119.888 111.506) (width 0.3048) (layer "F.Cu") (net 1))
 (segment (start 119.888 114.427) (end 119.888 113.157) (width 0.3048) (layer "F.Cu") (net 1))
 (segment (start 127.508 108.077) (end 133.096 108.077) (width 0.3048) (layer "F.Cu") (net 1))
 (segment (start 117.983 110.871) (end 118.618 111.506) (width 0.3048) (layer "F.Cu") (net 1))
 (segment (start 127.508 108.077) (end 130.429 108.077) (width 0.3048) (layer "F.Cu") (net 1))
 (segment (start 119.888 114.681) (end 120.523 115.316) (width 0.3) (layer "F.Cu") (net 1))
 (segment (start 127.508 109.347) (end 130.429 109.347) (width 0.3048) (layer "F.Cu") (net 1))
 (segment (start 136.271 108.966) (end 135.128 108.966) (width 0.3) (layer "F.Cu") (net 1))
 (segment (start 119.888 113.157) (end 119.888 111.506) (width 0.3048) (layer "F.Cu") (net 1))
 (segment (start 119.888 114.427) (end 119.888 114.681) (width 0.3) (layer "F.Cu") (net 1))
 (segment (start 133.096 109.347) (end 134.747 109.347) (width 0.3) (layer "F.Cu") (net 1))
 (segment (start 134.747 109.347) (end 135.128 108.966) (width 0.3) (layer "F.Cu") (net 1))
 (segment (start 127.508 108.077) (end 128.905 108.077) (width 0.3048) (layer "F.Cu") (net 1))
 (via (at 120.523 115.316) (size 0.9) (drill 0.5) (layers "F.Cu" "B.Cu") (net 1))
 (via (at 117.983 110.617) (size 0.9) (drill 0.5) (layers "F.Cu" "B.Cu") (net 1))
 (via (at 135.128 108.966) (size 0.9) (drill 0.5) (layers "F.Cu" "B.Cu") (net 1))
 (segment (start 114.554 110.617) (end 113.665 111.506) (width 0.3048) (layer "B.Cu") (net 1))
 (segment (start 113.665 114.554) (end 112.649 115.57) (width 0.3048) (layer "B.Cu") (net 1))
 (segment (start 112.649 115.57) (end 110.871 115.57) (width 0.3048) (layer "B.Cu") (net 1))
 (segment (start 110.871 115.57) (end 110.236 114.935) (width 0.3048) (layer "B.Cu") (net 1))
 (segment (start 110.236 114.935) (end 110.236 112.141) (width 0.3048) (layer "B.Cu") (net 1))
 (segment (start 110.236 112.141) (end 109.728 111.633) (width 0.3048) (layer "B.Cu") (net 1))
 (segment (start 109.728 111.633) (end 106.299 111.633) (width 0.3048) (layer "B.Cu") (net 1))
 (segment (start 106.299 111.633) (end 105.283 110.617) (width 0.3048) (layer "B.Cu") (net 1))
 (segment (start 105.283 110.617) (end 103.632 110.617) (width 0.3048) (layer "B.Cu") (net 1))
 (segment (start 113.665 111.506) (end 113.665 114.554) (width 0.3048) (layer "B.Cu") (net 1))
 (segment (start 115.824 110.617) (end 117.983 110.617) (width 0.3048) (layer "B.Cu") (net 1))
 (segment (start 133.731 110.6932) (end 133.731 109.474) (width 0.3) (layer "B.Cu") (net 1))
 (segment (start 121.9835 116.5225) (end 122.174 116.713) (width 0.3) (layer "B.Cu") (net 1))
 (segment (start 121.9835 115.316) (end 121.9962 115.3033) (width 0.3) (layer "B.Cu") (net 1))
 (segment (start 124.587 116.713) (end 125.984 118.11) (width 0.3) (layer "B.Cu") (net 1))
 (segment (start 120.523 115.316) (end 121.9835 115.316) (width 0.3) (layer "B.Cu") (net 1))
 (segment (start 122.174 116.713) (end 124.587 116.713) (width 0.3) (layer "B.Cu") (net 1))
 (segment (start 121.9835 115.316) (end 121.9835 116.5225) (width 0.3) (layer "B.Cu") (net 1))
 (segment (start 121.9962 115.3033) (end 121.9962 113.919) (width 0.3) (layer "B.Cu") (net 1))
 (segment (start 115.824 110.617) (end 114.554 110.617) (width 0.3048) (layer "B.Cu") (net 1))
 (segment (start 133.731 109.474) (end 134.239 108.966) (width 0.3) (layer "B.Cu") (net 1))
 (segment (start 134.239 108.966) (end 135.128 108.966) (width 0.3) (layer "B.Cu") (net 1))
 (segment (start 106.172 104.521) (end 107.696 106.045) (width 0.3048) (layer "F.Cu") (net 8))
 (segment (start 107.696 106.045) (end 109.601 106.045) (width 0.3048) (layer "F.Cu") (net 8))
 (segment (start 109.601 106.045) (end 110.617 107.061) (width 0.3048) (layer "F.Cu") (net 8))
 (segment (start 110.617 107.061) (end 110.617 108.458) (width 0.3048) (layer "F.Cu") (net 8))
 (segment (start 110.617 108.458) (end 112.776 110.617) (width 0.3048) (layer "F.Cu") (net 8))
 (segment (start 112.776 110.617) (end 114.681 110.617) (width 0.3048) (layer "F.Cu") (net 8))
 (segment (start 117.348 112.268) (end 116.84 111.76) (width 0.3048) (layer "F.Cu") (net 8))
 (segment (start 116.84 111.76) (end 115.824 111.76) (width 0.3048) (layer "F.Cu") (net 8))
 (segment (start 115.824 111.76) (end 114.681 110.617) (width 0.3048) (layer "F.Cu") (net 8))
 (segment (start 117.348 113.157) (end 117.348 112.268) (width 0.3048) (layer "F.Cu") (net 8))
 (segment (start 106.172 104.521) (end 106.172 103.632) (width 0.3048) (layer "F.Cu") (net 8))
 (segment (start 112.141 116.459) (end 111.252 117.348) (width 0.3048) (layer "F.Cu") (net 5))
 (segment (start 111.252 117.348) (end 111.252 118.618) (width 0.3048) (layer "F.Cu") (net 5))
 (via (at 112.141 116.459) (size 0.9) (drill 0.5) (layers "F.Cu" "B.Cu") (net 5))
 (segment (start 113.538 115.57) (end 114.935 115.57) (width 0.3048) (layer "B.Cu") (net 5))
 (segment (start 114.935 115.57) (end 115.189 115.316) (width 0.3048) (layer "B.Cu") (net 5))
 (segment (start 115.189 113.919) (end 115.189 115.316) (width 0.3048) (layer "B.Cu") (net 5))
 (segment (start 112.649 116.459) (end 112.141 116.459) (width 0.3048) (layer "B.Cu") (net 5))
 (segment (start 113.538 115.57) (end 112.649 116.459) (width 0.3048) (layer "B.Cu") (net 5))
 (segment (start 108.966 104.521) (end 111.252 106.807) (width 0.3048) (layer "F.Cu") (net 9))
 (segment (start 111.252 106.807) (end 111.252 108.204) (width 0.3048) (layer "F.Cu") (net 9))
 (segment (start 111.252 108.204) (end 113.03 109.982) (width 0.3048) (layer "F.Cu") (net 9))
 (segment (start 113.03 109.982) (end 114.935 109.982) (width 0.3048) (layer "F.Cu") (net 9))
 (segment (start 118.618 113.157) (end 118.618 112.268) (width 0.3048) (layer "F.Cu") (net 9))
 (segment (start 116.078 111.125) (end 117.094 111.125) (width 0.3048) (layer "F.Cu") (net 9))
 (segment (start 117.094 111.125) (end 117.983 112.014) (width 0.3048) (layer "F.Cu") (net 9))
 (segment (start 117.983 112.014) (end 118.364 112.014) (width 0.3048) (layer "F.Cu") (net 9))
 (segment (start 118.364 112.014) (end 118.618 112.268) (width 0.3048) (layer "F.Cu") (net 9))
 (segment (start 114.935 109.982) (end 116.078 111.125) (width 0.3048) (layer "F.Cu") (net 9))
 (segment (start 108.966 104.521) (end 108.966 103.632) (width 0.3048) (layer "F.Cu") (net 9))
 (segment (start 116.459 114.935) (end 118.872 114.935) (width 0.3048) (layer "F.Cu") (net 18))
 (segment (start 123.1265 113.919) (end 123.698 113.919) (width 0.3048) (layer "F.Cu") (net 18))
 (segment (start 116.078 113.157) (end 116.078 114.554) (width 0.3048) (layer "F.Cu") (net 18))
 (segment (start 116.078 114.554) (end 116.459 114.935) (width 0.3048) (layer "F.Cu") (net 18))
 (segment (start 120.142 116.205) (end 120.8405 116.205) (width 0.3048) (layer "F.Cu") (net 18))
 (segment (start 120.8405 116.205) (end 123.1265 113.919) (width 0.3048) (layer "F.Cu") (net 18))
 (segment (start 118.872 114.935) (end 120.142 116.205) (width 0.3048) (layer "F.Cu") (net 18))
 (via (at 123.698 113.919) (size 0.9) (drill 0.5) (layers "F.Cu" "B.Cu") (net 18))
 (segment (start 123.698 113.919) (end 125.349 113.919) (width 0.3048) (layer "B.Cu") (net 18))
 (segment (start 122.2375 107.569) (end 122.682 108.0135) (width 0.3048) (layer "F.Cu") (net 11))
 (segment (start 122.682 108.0135) (end 122.682 108.966) (width 0.3048) (layer "F.Cu") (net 11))
 (segment (start 121.158 107.569) (end 122.2375 107.569) (width 0.3048) (layer "F.Cu") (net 11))
 (via (at 122.682 108.966) (size 0.9) (drill 0.5) (layers "F.Cu" "B.Cu") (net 11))
 (segment (start 122.682 108.966) (end 122.682 110.109) (width 0.3048) (layer "B.Cu") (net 11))
 (segment (start 122.682 110.109) (end 123.19 110.617) (width 0.3048) (layer "B.Cu") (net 11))
 (segment (start 117.348 108.585) (end 117.348 107.569) (width 0.3048) (layer "F.Cu") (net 14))
 (segment (start 117.729 108.966) (end 117.348 108.585) (width 0.3048) (layer "F.Cu") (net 14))
 (via (at 117.729 108.966) (size 0.9) (drill 0.5) (layers "F.Cu" "B.Cu") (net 14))
 (segment (start 117.729 108.966) (end 117.729 107.823) (width 0.3048) (layer "B.Cu") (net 14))
 (segment (start 117.729 107.823) (end 117.221 107.315) (width 0.3048) (layer "B.Cu") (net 14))
 (segment (start 117.221 107.315) (end 115.824 107.315) (width 0.3048) (layer "B.Cu") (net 14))
 (segment (start 116.078 107.569) (end 116.078 108.966) (width 0.3048) (layer "F.Cu") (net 15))
 (via (at 116.078 108.966) (size 0.9) (drill 0.5) (layers "F.Cu" "B.Cu") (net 15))
 (segment (start 116.078 108.966) (end 114.9985 108.966) (width 0.3048) (layer "B.Cu") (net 15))
 (segment (start 114.9985 108.966) (end 113.3475 107.315) (width 0.3048) (layer "B.Cu") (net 15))
 (segment (start 113.3475 107.315) (end 112.268 107.315) (width 0.3048) (layer "B.Cu") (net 15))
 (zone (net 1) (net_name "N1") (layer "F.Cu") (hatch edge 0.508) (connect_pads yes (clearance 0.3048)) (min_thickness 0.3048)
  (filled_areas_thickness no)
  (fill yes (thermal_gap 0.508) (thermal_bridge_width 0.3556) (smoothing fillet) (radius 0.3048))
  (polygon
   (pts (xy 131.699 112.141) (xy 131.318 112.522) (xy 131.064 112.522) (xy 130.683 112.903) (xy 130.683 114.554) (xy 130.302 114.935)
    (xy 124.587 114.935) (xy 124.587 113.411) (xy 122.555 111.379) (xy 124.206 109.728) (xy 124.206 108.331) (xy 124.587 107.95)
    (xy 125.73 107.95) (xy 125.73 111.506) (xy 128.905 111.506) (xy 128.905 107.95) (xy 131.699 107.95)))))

